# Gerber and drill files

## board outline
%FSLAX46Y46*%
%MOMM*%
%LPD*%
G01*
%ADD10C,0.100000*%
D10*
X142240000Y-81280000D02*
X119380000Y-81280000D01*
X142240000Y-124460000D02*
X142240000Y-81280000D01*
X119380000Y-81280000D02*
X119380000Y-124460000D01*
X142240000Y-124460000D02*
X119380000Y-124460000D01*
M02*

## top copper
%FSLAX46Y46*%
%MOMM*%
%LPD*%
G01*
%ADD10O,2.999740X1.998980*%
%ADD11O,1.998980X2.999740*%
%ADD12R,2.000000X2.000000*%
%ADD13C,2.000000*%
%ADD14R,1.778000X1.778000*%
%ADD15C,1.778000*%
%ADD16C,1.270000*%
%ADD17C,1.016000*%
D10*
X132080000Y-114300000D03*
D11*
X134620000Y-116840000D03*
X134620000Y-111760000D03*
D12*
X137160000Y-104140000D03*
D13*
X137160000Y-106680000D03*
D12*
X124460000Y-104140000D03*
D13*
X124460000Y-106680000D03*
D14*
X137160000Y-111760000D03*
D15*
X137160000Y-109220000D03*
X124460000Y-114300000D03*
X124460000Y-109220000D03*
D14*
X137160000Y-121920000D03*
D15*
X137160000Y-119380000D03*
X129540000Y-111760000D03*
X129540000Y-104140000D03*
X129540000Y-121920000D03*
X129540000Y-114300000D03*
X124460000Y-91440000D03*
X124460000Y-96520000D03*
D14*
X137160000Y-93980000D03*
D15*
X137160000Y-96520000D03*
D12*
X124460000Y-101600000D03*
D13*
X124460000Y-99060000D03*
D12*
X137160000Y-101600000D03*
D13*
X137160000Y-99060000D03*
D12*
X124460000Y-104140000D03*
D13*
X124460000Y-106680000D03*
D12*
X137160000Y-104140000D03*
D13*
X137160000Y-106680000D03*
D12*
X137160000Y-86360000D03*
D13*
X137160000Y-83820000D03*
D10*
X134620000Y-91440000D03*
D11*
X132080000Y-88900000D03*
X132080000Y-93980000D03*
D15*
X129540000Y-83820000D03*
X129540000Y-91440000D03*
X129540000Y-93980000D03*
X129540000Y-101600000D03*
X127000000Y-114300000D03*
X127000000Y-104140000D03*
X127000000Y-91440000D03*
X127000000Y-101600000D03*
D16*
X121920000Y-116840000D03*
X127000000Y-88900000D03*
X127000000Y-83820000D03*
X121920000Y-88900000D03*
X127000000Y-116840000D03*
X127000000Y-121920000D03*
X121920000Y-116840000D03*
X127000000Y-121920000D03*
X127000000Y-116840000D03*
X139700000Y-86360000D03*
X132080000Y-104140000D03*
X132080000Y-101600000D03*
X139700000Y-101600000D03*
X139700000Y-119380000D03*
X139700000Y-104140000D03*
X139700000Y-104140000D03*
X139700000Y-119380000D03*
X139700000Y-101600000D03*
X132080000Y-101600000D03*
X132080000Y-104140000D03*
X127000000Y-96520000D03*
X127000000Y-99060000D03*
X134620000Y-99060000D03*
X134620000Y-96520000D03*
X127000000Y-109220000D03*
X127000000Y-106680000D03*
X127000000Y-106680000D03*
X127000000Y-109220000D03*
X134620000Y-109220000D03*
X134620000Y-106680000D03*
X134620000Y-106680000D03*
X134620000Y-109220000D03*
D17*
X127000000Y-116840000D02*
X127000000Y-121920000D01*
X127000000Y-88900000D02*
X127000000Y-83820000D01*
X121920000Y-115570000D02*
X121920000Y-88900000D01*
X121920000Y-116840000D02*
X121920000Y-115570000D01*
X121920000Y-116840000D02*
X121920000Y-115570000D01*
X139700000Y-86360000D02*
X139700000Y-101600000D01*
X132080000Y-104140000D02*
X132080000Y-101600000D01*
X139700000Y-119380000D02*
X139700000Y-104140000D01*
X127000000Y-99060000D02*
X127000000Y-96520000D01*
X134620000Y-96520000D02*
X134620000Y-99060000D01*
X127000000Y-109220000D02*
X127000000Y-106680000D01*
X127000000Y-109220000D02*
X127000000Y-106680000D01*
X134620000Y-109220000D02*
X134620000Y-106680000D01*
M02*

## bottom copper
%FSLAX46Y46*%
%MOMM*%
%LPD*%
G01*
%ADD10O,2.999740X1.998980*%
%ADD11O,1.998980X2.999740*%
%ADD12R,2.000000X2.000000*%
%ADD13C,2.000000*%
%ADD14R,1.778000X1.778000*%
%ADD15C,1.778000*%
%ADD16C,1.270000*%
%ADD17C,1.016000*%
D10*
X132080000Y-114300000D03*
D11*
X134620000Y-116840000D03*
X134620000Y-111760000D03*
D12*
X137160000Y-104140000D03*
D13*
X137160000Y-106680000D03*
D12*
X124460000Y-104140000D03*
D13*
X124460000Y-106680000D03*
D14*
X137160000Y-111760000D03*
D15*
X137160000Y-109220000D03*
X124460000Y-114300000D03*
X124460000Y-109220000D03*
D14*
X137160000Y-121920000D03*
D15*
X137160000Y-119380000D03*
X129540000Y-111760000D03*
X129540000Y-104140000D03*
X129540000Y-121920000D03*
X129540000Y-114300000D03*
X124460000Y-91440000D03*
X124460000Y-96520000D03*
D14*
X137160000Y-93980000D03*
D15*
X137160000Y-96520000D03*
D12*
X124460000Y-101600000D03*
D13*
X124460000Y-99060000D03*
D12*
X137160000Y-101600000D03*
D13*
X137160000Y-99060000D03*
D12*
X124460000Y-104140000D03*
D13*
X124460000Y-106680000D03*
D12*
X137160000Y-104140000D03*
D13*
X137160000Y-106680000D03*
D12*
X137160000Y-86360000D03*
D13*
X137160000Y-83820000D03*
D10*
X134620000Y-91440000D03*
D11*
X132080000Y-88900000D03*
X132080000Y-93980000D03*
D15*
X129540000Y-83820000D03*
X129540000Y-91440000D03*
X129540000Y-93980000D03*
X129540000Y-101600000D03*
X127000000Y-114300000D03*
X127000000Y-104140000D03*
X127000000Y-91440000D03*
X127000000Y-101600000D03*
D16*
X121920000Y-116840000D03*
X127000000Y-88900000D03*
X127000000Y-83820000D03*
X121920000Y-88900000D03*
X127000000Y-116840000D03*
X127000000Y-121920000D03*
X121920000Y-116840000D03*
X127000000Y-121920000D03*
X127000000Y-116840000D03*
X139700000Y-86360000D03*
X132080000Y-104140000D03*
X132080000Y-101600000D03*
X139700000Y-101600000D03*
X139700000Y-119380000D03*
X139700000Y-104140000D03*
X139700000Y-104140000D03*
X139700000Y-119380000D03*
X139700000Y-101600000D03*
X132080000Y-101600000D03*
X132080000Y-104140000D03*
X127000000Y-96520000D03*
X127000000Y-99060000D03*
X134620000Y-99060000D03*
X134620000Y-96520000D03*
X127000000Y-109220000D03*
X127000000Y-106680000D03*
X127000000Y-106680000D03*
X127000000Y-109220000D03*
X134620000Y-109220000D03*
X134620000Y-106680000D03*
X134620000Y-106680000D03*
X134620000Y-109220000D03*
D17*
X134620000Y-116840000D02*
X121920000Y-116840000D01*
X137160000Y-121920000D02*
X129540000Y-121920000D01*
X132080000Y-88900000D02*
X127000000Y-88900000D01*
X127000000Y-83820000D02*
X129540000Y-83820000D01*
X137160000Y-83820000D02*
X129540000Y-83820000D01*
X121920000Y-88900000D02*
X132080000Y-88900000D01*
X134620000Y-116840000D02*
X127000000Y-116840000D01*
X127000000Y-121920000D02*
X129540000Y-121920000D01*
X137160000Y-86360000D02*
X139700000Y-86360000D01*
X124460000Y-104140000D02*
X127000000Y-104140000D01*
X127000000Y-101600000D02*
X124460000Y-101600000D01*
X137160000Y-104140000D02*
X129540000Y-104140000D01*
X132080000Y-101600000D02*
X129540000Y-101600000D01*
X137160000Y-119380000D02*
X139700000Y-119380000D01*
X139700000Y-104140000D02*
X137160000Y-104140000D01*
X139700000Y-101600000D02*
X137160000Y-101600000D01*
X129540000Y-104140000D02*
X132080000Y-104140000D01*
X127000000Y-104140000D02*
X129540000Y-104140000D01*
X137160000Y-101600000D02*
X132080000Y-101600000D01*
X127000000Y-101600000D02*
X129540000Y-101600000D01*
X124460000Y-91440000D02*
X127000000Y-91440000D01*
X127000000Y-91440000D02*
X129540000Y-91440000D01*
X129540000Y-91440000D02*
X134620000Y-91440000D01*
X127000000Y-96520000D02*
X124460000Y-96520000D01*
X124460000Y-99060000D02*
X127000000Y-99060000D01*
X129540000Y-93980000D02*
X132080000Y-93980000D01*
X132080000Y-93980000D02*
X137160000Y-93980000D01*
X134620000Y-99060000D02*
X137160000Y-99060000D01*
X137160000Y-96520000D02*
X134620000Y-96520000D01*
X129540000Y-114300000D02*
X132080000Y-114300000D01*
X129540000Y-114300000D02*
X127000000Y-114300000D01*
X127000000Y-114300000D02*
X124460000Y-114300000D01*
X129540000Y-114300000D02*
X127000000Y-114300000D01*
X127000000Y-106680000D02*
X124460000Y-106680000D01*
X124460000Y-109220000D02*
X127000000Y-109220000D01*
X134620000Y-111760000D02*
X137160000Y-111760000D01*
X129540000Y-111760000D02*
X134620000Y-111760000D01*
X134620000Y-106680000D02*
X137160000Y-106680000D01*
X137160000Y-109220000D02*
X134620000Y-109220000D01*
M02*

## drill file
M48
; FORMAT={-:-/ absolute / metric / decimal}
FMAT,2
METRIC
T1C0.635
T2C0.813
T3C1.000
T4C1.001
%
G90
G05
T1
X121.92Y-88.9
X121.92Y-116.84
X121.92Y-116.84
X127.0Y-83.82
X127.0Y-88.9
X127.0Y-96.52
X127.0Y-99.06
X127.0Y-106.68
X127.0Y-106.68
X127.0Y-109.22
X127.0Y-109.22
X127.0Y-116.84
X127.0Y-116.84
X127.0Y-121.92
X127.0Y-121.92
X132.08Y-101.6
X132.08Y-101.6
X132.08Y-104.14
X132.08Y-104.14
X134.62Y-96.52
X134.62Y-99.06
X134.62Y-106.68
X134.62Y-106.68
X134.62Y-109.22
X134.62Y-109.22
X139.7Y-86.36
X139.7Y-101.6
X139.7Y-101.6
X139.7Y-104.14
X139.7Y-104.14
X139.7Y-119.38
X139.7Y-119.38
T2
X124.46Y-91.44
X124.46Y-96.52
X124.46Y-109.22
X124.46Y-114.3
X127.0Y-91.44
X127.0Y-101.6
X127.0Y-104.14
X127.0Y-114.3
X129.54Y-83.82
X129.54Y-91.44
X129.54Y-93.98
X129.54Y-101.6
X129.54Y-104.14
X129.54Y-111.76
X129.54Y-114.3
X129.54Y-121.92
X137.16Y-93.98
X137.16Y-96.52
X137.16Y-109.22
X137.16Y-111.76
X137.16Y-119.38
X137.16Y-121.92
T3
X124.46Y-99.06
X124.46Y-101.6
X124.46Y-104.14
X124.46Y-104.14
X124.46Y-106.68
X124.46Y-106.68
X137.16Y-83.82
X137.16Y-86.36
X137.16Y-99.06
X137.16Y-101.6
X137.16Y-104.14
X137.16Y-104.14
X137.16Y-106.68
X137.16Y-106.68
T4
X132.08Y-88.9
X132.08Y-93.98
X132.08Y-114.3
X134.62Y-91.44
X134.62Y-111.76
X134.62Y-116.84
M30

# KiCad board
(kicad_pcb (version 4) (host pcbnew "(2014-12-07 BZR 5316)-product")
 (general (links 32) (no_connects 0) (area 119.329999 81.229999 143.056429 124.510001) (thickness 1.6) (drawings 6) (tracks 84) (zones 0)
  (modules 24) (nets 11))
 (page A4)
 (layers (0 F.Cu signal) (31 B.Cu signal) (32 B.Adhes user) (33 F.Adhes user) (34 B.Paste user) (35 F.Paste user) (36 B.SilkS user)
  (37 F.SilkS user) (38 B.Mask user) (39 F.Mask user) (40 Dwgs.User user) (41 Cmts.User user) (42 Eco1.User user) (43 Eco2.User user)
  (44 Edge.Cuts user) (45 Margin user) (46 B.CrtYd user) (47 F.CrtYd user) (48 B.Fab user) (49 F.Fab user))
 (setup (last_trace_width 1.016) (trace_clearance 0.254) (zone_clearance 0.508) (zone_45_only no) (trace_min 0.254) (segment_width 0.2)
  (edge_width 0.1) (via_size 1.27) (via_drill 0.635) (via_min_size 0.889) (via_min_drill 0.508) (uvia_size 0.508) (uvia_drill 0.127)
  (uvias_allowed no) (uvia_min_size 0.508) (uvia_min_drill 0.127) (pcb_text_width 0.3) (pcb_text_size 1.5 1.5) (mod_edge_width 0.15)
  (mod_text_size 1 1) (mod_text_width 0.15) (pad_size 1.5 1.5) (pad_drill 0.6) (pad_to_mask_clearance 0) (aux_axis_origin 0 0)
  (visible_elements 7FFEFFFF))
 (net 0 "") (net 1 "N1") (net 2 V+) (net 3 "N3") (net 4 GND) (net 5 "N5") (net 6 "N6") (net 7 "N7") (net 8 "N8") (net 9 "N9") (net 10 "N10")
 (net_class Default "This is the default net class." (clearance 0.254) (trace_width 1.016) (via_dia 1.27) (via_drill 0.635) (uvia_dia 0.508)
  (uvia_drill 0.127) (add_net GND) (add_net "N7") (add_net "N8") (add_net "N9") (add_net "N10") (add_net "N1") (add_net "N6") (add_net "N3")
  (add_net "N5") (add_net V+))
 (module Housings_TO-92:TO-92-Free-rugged (layer F.Cu) (at 134.62 114.3 180)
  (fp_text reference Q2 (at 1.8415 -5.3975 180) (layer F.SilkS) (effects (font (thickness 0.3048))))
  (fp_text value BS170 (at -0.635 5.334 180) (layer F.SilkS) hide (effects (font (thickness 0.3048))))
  (pad 2 thru_hole oval (at 2.54 0 180) (size 2.99974 1.99898) (drill 1.00076) (layers *.Cu *.Mask F.SilkS) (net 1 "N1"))
  (pad 1 thru_hole oval (at 0 -2.54 180) (size 1.99898 2.99974) (drill 1.00076) (layers *.Cu *.Mask F.SilkS) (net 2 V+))
  (pad 3 thru_hole oval (at 0 2.54 180) (size 1.99898 2.99974) (drill 1.00076) (layers *.Cu *.Mask F.SilkS) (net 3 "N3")))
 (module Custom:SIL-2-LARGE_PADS (layer F.Cu) (at 137.16 105.41 270)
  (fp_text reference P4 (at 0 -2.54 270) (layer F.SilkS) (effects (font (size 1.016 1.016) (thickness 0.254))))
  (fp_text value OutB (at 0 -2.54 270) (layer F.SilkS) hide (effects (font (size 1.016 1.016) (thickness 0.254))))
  (pad 1 thru_hole rect (at -1.27 0 270) (size 2 2) (drill 1) (layers *.Cu *.Mask F.SilkS) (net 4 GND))
  (pad 2 thru_hole circle (at 1.27 0 270) (size 2 2) (drill 1) (layers *.Cu *.Mask F.SilkS) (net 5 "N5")))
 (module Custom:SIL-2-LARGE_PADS (layer F.Cu) (at 124.46 105.41 270)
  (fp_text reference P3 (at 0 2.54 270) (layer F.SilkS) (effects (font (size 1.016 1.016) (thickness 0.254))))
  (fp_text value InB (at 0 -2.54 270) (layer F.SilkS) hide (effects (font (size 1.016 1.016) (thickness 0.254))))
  (pad 1 thru_hole rect (at -1.27 0 270) (size 2 2) (drill 1) (layers *.Cu *.Mask F.SilkS) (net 4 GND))
  (pad 2 thru_hole circle (at 1.27 0 270) (size 2 2) (drill 1) (layers *.Cu *.Mask F.SilkS) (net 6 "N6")))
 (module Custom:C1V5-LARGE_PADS (layer F.Cu) (at 137.16 110.49 90)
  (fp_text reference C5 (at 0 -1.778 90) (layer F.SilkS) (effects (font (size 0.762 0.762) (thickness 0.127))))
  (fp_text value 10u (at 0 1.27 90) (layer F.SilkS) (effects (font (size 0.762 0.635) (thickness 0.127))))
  (pad 1 thru_hole rect (at -1.27 0 90) (size 1.778 1.778) (drill 0.8128) (layers *.Cu *.Mask F.SilkS) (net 3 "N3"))
  (pad 2 thru_hole circle (at 1.27 0 90) (size 1.778 1.778) (drill 0.8128) (layers *.Cu *.Mask F.SilkS) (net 5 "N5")))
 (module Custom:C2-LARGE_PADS (layer F.Cu) (at 124.46 111.76 90)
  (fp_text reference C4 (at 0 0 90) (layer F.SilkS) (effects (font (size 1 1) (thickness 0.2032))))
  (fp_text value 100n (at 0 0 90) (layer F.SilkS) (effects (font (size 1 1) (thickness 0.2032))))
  (pad 1 thru_hole circle (at -2.54 0 90) (size 1.778 1.778) (drill 0.8128) (layers *.Cu *.Mask F.SilkS) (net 1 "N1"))
  (pad 2 thru_hole circle (at 2.54 0 90) (size 1.778 1.778) (drill 0.8128) (layers *.Cu *.Mask F.SilkS) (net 6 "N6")))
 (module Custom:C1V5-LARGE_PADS (layer F.Cu) (at 137.16 120.65 90)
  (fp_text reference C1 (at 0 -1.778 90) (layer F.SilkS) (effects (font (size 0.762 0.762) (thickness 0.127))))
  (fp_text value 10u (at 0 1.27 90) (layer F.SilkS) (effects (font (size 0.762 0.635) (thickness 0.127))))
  (pad 1 thru_hole rect (at -1.27 0 90) (size 1.778 1.778) (drill 0.8128) (layers *.Cu *.Mask F.SilkS) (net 2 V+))
  (pad 2 thru_hole circle (at 1.27 0 90) (size 1.778 1.778) (drill 0.8128) (layers *.Cu *.Mask F.SilkS) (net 4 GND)))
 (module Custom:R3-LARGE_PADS (layer F.Cu) (at 129.54 107.95 90) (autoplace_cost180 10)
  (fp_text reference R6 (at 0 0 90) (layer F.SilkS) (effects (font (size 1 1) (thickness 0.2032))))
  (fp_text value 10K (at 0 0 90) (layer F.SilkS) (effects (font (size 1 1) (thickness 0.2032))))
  (pad 1 thru_hole circle (at -3.81 0 90) (size 1.778 1.778) (drill 0.8128) (layers *.Cu *.Mask F.SilkS) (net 3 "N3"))
  (pad 2 thru_hole circle (at 3.81 0 90) (size 1.778 1.778) (drill 0.8128) (layers *.Cu *.Mask F.SilkS) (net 4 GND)))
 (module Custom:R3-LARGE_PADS (layer F.Cu) (at 129.54 118.11 90) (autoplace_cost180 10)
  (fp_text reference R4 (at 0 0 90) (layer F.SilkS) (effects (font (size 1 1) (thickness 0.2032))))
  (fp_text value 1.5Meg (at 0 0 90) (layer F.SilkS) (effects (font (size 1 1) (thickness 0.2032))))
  (pad 1 thru_hole circle (at -3.81 0 90) (size 1.778 1.778) (drill 0.8128) (layers *.Cu *.Mask F.SilkS) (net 2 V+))
  (pad 2 thru_hole circle (at 3.81 0 90) (size 1.778 1.778) (drill 0.8128) (layers *.Cu *.Mask F.SilkS) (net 1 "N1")))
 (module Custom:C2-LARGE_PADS (layer F.Cu) (at 124.46 93.98 270)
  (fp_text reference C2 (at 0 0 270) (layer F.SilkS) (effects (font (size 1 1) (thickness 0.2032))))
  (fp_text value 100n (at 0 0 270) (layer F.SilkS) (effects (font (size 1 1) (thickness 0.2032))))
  (pad 1 thru_hole circle (at -2.54 0 270) (size 1.778 1.778) (drill 0.8128) (layers *.Cu *.Mask F.SilkS) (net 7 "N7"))
  (pad 2 thru_hole circle (at 2.54 0 270) (size 1.778 1.778) (drill 0.8128) (layers *.Cu *.Mask F.SilkS) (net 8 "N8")))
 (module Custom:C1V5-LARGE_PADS (layer F.Cu) (at 137.16 95.25 270)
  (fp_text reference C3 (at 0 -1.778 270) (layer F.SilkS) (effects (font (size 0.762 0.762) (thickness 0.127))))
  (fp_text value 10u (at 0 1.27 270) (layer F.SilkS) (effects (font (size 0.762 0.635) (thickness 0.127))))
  (pad 1 thru_hole rect (at -1.27 0 270) (size 1.778 1.778) (drill 0.8128) (layers *.Cu *.Mask F.SilkS) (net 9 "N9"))
  (pad 2 thru_hole circle (at 1.27 0 270) (size 1.778 1.778) (drill 0.8128) (layers *.Cu *.Mask F.SilkS) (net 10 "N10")))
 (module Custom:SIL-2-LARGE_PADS (layer F.Cu) (at 124.46 100.33 90)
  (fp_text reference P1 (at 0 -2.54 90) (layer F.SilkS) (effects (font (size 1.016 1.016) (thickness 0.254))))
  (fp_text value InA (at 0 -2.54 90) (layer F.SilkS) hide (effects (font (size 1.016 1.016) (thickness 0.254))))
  (pad 1 thru_hole rect (at -1.27 0 90) (size 2 2) (drill 1) (layers *.Cu *.Mask F.SilkS) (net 4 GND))
  (pad 2 thru_hole circle (at 1.27 0 90) (size 2 2) (drill 1) (layers *.Cu *.Mask F.SilkS) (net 8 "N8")))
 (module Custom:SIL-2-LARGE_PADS (layer F.Cu) (at 137.16 100.33 90)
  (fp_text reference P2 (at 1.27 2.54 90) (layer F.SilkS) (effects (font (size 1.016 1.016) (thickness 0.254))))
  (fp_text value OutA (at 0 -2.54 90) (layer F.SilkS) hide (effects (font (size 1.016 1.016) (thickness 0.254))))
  (pad 1 thru_hole rect (at -1.27 0 90) (size 2 2) (drill 1) (layers *.Cu *.Mask F.SilkS) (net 4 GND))
  (pad 2 thru_hole circle (at 1.27 0 90) (size 2 2) (drill 1) (layers *.Cu *.Mask F.SilkS) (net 10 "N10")))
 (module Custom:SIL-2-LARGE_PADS (layer F.Cu) (at 124.46 105.41 270)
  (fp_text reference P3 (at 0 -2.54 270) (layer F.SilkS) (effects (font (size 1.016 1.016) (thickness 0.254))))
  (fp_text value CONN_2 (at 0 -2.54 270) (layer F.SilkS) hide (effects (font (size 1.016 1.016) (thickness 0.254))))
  (pad 1 thru_hole rect (at -1.27 0 270) (size 2 2) (drill 1) (layers *.Cu *.Mask F.SilkS) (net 4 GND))
  (pad 2 thru_hole circle (at 1.27 0 270) (size 2 2) (drill 1) (layers *.Cu *.Mask F.SilkS) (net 6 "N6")))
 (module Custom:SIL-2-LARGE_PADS (layer F.Cu) (at 137.16 105.41 270)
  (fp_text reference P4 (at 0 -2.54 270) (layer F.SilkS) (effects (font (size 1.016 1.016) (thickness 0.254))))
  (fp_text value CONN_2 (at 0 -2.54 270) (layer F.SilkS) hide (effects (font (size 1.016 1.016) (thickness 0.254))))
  (pad 1 thru_hole rect (at -1.27 0 270) (size 2 2) (drill 1) (layers *.Cu *.Mask F.SilkS) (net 4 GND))
  (pad 2 thru_hole circle (at 1.27 0 270) (size 2 2) (drill 1) (layers *.Cu *.Mask F.SilkS) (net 5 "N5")))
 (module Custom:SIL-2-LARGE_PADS (layer F.Cu) (at 137.16 85.09 90)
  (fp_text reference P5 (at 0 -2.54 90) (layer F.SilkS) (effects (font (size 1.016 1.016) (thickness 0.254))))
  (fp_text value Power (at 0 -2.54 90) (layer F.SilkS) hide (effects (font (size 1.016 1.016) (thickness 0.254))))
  (pad 1 thru_hole rect (at -1.27 0 90) (size 2 2) (drill 1) (layers *.Cu *.Mask F.SilkS) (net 4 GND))
  (pad 2 thru_hole circle (at 1.27 0 90) (size 2 2) (drill 1) (layers *.Cu *.Mask F.SilkS) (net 2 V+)))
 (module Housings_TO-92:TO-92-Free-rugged (layer F.Cu) (at 132.08 91.44)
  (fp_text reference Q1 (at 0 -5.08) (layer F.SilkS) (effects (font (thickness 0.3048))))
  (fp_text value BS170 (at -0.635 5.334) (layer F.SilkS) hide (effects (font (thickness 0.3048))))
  (pad 2 thru_hole oval (at 2.54 0) (size 2.99974 1.99898) (drill 1.00076) (layers *.Cu *.Mask F.SilkS) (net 7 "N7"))
  (pad 1 thru_hole oval (at 0 -2.54) (size 1.99898 2.99974) (drill 1.00076) (layers *.Cu *.Mask F.SilkS) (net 2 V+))
  (pad 3 thru_hole oval (at 0 2.54) (size 1.99898 2.99974) (drill 1.00076) (layers *.Cu *.Mask F.SilkS) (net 9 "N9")))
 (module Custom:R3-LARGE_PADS (layer F.Cu) (at 129.54 87.63 270) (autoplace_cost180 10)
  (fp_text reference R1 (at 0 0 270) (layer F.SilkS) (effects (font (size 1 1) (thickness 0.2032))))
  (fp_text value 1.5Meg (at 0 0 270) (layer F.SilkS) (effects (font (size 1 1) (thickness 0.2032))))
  (pad 1 thru_hole circle (at -3.81 0 270) (size 1.778 1.778) (drill 0.8128) (layers *.Cu *.Mask F.SilkS) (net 2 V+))
  (pad 2 thru_hole circle (at 3.81 0 270) (size 1.778 1.778) (drill 0.8128) (layers *.Cu *.Mask F.SilkS) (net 7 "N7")))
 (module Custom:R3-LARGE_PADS (layer F.Cu) (at 129.54 97.79 270) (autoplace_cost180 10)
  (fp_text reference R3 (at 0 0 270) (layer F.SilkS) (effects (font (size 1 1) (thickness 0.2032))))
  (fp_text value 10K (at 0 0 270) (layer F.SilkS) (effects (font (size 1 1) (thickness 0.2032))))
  (pad 1 thru_hole circle (at -3.81 0 270) (size 1.778 1.778) (drill 0.8128) (layers *.Cu *.Mask F.SilkS) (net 9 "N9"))
  (pad 2 thru_hole circle (at 3.81 0 270) (size 1.778 1.778) (drill 0.8128) (layers *.Cu *.Mask F.SilkS) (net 4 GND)))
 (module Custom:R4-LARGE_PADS (layer F.Cu) (at 127 109.22 90) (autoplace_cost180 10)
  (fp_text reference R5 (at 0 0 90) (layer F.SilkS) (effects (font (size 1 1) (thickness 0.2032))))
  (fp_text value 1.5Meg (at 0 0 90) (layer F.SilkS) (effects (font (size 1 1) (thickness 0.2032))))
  (pad 1 thru_hole circle (at -5.08 0 90) (size 1.778 1.778) (drill 0.8128) (layers *.Cu *.Mask F.SilkS) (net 1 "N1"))
  (pad 2 thru_hole circle (at 5.08 0 90) (size 1.778 1.778) (drill 0.8128) (layers *.Cu *.Mask F.SilkS) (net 4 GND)))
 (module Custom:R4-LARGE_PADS (layer F.Cu) (at 127 96.52 270) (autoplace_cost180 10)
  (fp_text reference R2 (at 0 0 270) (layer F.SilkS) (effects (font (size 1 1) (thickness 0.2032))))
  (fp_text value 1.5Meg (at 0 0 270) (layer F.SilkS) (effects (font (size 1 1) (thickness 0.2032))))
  (pad 1 thru_hole circle (at -5.08 0 270) (size 1.778 1.778) (drill 0.8128) (layers *.Cu *.Mask F.SilkS) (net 7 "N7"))
  (pad 2 thru_hole circle (at 5.08 0 270) (size 1.778 1.778) (drill 0.8128) (layers *.Cu *.Mask F.SilkS) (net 4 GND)))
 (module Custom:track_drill (layer F.Cu) (at 132.08 96.52)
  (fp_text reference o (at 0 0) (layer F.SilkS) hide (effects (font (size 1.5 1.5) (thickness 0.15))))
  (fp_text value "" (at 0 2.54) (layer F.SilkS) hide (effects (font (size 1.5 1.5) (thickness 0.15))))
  (pad 1 connect rect (at 0 0 45) (size 1.524 1.524) (layers *.Mask B.SilkS Dwgs.User) (die_length 0.254)))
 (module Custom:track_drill (layer F.Cu) (at 132.08 99.06)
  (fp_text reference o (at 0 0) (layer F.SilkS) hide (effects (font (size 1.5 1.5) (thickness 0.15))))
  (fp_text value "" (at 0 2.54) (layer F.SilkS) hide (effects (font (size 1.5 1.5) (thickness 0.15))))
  (pad 1 connect rect (at 0 0 45) (size 1.524 1.524) (layers *.Mask B.SilkS Dwgs.User) (die_length 0.254)))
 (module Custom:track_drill (layer F.Cu) (at 132.08 106.68)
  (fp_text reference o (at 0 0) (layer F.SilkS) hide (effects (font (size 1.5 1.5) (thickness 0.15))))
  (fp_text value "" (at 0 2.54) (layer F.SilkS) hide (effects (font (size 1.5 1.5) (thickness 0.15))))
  (pad 1 connect rect (at 0 0 45) (size 1.524 1.524) (layers *.Mask B.SilkS Dwgs.User) (die_length 0.254)))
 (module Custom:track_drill (layer F.Cu) (at 132.08 109.22)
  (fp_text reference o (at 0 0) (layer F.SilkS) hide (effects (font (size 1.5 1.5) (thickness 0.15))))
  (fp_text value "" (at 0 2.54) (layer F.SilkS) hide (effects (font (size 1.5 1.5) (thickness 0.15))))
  (pad 1 connect rect (at 0 0 45) (size 1.524 1.524) (layers *.Mask B.SilkS Dwgs.User) (die_length 0.254)))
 (gr_line (start 142.24 81.28) (end 119.38 81.28) (angle 90) (layer Edge.Cuts) (width 0.1))
 (gr_line (start 142.24 124.46) (end 142.24 81.28) (angle 90) (layer Edge.Cuts) (width 0.1))
 (gr_line (start 119.38 81.28) (end 119.38 124.46) (angle 90) (layer Edge.Cuts) (width 0.1))
 (gr_line (start 142.24 124.46) (end 119.38 124.46) (angle 90) (layer Edge.Cuts) (width 0.1))
 (via (at 121.92 116.84) (size 1.27) (layers F.Cu B.Cu) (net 2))
 (segment (start 134.62 116.84) (end 121.92 116.84) (width 1.016) (layer B.Cu) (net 2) (status 10))
 (segment (start 127 116.84) (end 127 121.92) (width 1.016) (layer F.Cu) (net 2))
 (segment (start 137.16 121.92) (end 129.54 121.92) (width 1.016) (layer B.Cu) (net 2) (status 30))
 (segment (start 132.08 88.9) (end 127 88.9) (width 1.016) (layer B.Cu) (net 2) (status 10))
 (via (at 127 88.9) (size 1.27) (layers F.Cu B.Cu) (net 2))
 (segment (start 127 88.9) (end 127 83.82) (width 1.016) (layer F.Cu) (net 2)) (via (at 127 83.82) (size 1.27) (layers F.Cu B.Cu) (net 2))
 (segment (start 127 83.82) (end 129.54 83.82) (width 1.016) (layer B.Cu) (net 2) (status 20))
 (segment (start 137.16 83.82) (end 129.54 83.82) (width 1.016) (layer B.Cu) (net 2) (status 30))
 (segment (start 121.92 88.9) (end 132.08 88.9) (width 1.016) (layer B.Cu) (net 2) (status 20))
 (via (at 121.92 88.9) (size 1.27) (layers F.Cu B.Cu) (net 2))
 (segment (start 121.92 115.57) (end 121.92 88.9) (width 1.016) (layer F.Cu) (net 2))
 (via (at 127 116.84) (size 1.27) (layers F.Cu B.Cu) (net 2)) (via (at 127 121.92) (size 1.27) (layers F.Cu B.Cu) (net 2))
 (segment (start 134.62 116.84) (end 127 116.84) (width 1.016) (layer B.Cu) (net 2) (status 10))
 (segment (start 121.92 116.84) (end 121.92 115.57) (width 1.016) (layer F.Cu) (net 2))
 (segment (start 121.92 116.84) (end 121.92 115.57) (width 1.016) (layer F.Cu) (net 2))
 (via (at 121.92 116.84) (size 1.27) (layers F.Cu B.Cu) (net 2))
 (segment (start 127 121.92) (end 129.54 121.92) (width 1.016) (layer B.Cu) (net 2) (status 20))
 (via (at 127 121.92) (size 1.27) (layers F.Cu B.Cu) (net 2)) (via (at 127 116.84) (size 1.27) (layers F.Cu B.Cu) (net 2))
 (segment (start 137.16 86.36) (end 139.7 86.36) (width 1.016) (layer B.Cu) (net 4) (status 10))
 (via (at 139.7 86.36) (size 1.27) (layers F.Cu B.Cu) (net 4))
 (segment (start 139.7 86.36) (end 139.7 101.6) (width 1.016) (layer F.Cu) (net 4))
 (segment (start 132.08 104.14) (end 132.08 101.6) (width 1.016) (layer F.Cu) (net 4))
 (segment (start 124.46 104.14) (end 127 104.14) (width 1.016) (layer B.Cu) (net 4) (status 30))
 (segment (start 127 101.6) (end 124.46 101.6) (width 1.016) (layer B.Cu) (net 4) (status 30))
 (segment (start 137.16 104.14) (end 129.54 104.14) (width 1.016) (layer B.Cu) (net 4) (status 30))
 (segment (start 132.08 101.6) (end 129.54 101.6) (width 1.016) (layer B.Cu) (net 4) (status 20))
 (via (at 132.08 104.14) (size 1.27) (layers F.Cu B.Cu) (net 4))
 (via (at 132.08 101.6) (size 1.27) (layers F.Cu B.Cu) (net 4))
 (via (at 139.7 101.6) (size 1.27) (layers F.Cu B.Cu) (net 4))
 (via (at 139.7 119.38) (size 1.27) (layers F.Cu B.Cu) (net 4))
 (via (at 139.7 104.14) (size 1.27) (layers F.Cu B.Cu) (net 4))
 (segment (start 137.16 119.38) (end 139.7 119.38) (width 1.016) (layer B.Cu) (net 4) (status 10))
 (segment (start 139.7 104.14) (end 137.16 104.14) (width 1.016) (layer B.Cu) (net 4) (status 20))
 (via (at 139.7 104.14) (size 1.27) (layers F.Cu B.Cu) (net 4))
 (segment (start 139.7 119.38) (end 139.7 104.14) (width 1.016) (layer F.Cu) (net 4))
 (via (at 139.7 119.38) (size 1.27) (layers F.Cu B.Cu) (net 4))
 (via (at 139.7 101.6) (size 1.27) (layers F.Cu B.Cu) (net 4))
 (segment (start 139.7 101.6) (end 137.16 101.6) (width 1.016) (layer B.Cu) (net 4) (status 20))
 (segment (start 129.54 104.14) (end 132.08 104.14) (width 1.016) (layer B.Cu) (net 4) (status 10))
 (via (at 132.08 101.6) (size 1.27) (layers F.Cu B.Cu) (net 4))
 (via (at 132.08 104.14) (size 1.27) (layers F.Cu B.Cu) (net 4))
 (segment (start 127 104.14) (end 129.54 104.14) (width 1.016) (layer B.Cu) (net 4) (status 30))
 (segment (start 137.16 101.6) (end 132.08 101.6) (width 1.016) (layer B.Cu) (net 4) (status 10))
 (segment (start 127 101.6) (end 129.54 101.6) (width 1.016) (layer B.Cu) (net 4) (status 30))
 (segment (start 124.46 91.44) (end 127 91.44) (width 1.016) (layer B.Cu) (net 7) (status 30))
 (segment (start 127 91.44) (end 129.54 91.44) (width 1.016) (layer B.Cu) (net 7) (status 30))
 (segment (start 129.54 91.44) (end 134.62 91.44) (width 1.016) (layer B.Cu) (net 7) (status 30))
 (segment (start 127 96.52) (end 124.46 96.52) (width 1.016) (layer B.Cu) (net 8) (status 20))
 (via (at 127 96.52) (size 1.27) (layers F.Cu B.Cu) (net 8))
 (segment (start 124.46 99.06) (end 127 99.06) (width 1.016) (layer B.Cu) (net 8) (status 10))
 (segment (start 127 99.06) (end 127 96.52) (width 1.016) (layer F.Cu) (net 8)) (via (at 127 99.06) (size 1.27) (layers F.Cu B.Cu) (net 8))
 (segment (start 129.54 93.98) (end 132.08 93.98) (width 1.016) (layer B.Cu) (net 9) (status 30))
 (segment (start 132.08 93.98) (end 137.16 93.98) (width 1.016) (layer B.Cu) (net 9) (status 30))
 (segment (start 134.62 99.06) (end 137.16 99.06) (width 1.016) (layer B.Cu) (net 10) (status 20))
 (segment (start 137.16 96.52) (end 134.62 96.52) (width 1.016) (layer B.Cu) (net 10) (status 10))
 (via (at 134.62 99.06) (size 1.27) (layers F.Cu B.Cu) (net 10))
 (segment (start 134.62 96.52) (end 134.62 99.06) (width 1.016) (layer F.Cu) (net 10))
 (via (at 134.62 96.52) (size 1.27) (layers F.Cu B.Cu) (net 10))
 (segment (start 129.54 114.3) (end 132.08 114.3) (width 1.016) (layer B.Cu) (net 1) (status 30))
 (segment (start 129.54 114.3) (end 127 114.3) (width 1.016) (layer B.Cu) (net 1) (status 30))
 (segment (start 127 114.3) (end 124.46 114.3) (width 1.016) (layer B.Cu) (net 1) (status 30))
 (segment (start 129.54 114.3) (end 127 114.3) (width 1.016) (layer B.Cu) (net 1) (status 30))
 (via (at 127 109.22) (size 1.27) (layers F.Cu B.Cu) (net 6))
 (segment (start 127 109.22) (end 127 106.68) (width 1.016) (layer F.Cu) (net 6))
 (via (at 127 106.68) (size 1.27) (layers F.Cu B.Cu) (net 6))
 (segment (start 127 106.68) (end 124.46 106.68) (width 1.016) (layer B.Cu) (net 6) (status 20))
 (segment (start 124.46 109.22) (end 127 109.22) (width 1.016) (layer B.Cu) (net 6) (status 10))
 (via (at 127 106.68) (size 1.27) (layers F.Cu B.Cu) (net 6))
 (segment (start 127 109.22) (end 127 106.68) (width 1.016) (layer F.Cu) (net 6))
 (via (at 127 109.22) (size 1.27) (layers F.Cu B.Cu) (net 6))
 (segment (start 134.62 111.76) (end 137.16 111.76) (width 1.016) (layer B.Cu) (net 3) (status 30))
 (segment (start 129.54 111.76) (end 134.62 111.76) (width 1.016) (layer B.Cu) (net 3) (status 30))
 (via (at 134.62 109.22) (size 1.27) (layers F.Cu B.Cu) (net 5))
 (via (at 134.62 106.68) (size 1.27) (layers F.Cu B.Cu) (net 5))
 (segment (start 134.62 106.68) (end 137.16 106.68) (width 1.016) (layer B.Cu) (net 5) (status 20))
 (segment (start 137.16 109.22) (end 134.62 109.22) (width 1.016) (layer B.Cu) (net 5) (status 10))
 (via (at 134.62 106.68) (size 1.27) (layers F.Cu B.Cu) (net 5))
 (segment (start 134.62 109.22) (end 134.62 106.68) (width 1.016) (layer F.Cu) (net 5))
 (via (at 134.62 109.22) (size 1.27) (layers F.Cu B.Cu) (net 5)))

